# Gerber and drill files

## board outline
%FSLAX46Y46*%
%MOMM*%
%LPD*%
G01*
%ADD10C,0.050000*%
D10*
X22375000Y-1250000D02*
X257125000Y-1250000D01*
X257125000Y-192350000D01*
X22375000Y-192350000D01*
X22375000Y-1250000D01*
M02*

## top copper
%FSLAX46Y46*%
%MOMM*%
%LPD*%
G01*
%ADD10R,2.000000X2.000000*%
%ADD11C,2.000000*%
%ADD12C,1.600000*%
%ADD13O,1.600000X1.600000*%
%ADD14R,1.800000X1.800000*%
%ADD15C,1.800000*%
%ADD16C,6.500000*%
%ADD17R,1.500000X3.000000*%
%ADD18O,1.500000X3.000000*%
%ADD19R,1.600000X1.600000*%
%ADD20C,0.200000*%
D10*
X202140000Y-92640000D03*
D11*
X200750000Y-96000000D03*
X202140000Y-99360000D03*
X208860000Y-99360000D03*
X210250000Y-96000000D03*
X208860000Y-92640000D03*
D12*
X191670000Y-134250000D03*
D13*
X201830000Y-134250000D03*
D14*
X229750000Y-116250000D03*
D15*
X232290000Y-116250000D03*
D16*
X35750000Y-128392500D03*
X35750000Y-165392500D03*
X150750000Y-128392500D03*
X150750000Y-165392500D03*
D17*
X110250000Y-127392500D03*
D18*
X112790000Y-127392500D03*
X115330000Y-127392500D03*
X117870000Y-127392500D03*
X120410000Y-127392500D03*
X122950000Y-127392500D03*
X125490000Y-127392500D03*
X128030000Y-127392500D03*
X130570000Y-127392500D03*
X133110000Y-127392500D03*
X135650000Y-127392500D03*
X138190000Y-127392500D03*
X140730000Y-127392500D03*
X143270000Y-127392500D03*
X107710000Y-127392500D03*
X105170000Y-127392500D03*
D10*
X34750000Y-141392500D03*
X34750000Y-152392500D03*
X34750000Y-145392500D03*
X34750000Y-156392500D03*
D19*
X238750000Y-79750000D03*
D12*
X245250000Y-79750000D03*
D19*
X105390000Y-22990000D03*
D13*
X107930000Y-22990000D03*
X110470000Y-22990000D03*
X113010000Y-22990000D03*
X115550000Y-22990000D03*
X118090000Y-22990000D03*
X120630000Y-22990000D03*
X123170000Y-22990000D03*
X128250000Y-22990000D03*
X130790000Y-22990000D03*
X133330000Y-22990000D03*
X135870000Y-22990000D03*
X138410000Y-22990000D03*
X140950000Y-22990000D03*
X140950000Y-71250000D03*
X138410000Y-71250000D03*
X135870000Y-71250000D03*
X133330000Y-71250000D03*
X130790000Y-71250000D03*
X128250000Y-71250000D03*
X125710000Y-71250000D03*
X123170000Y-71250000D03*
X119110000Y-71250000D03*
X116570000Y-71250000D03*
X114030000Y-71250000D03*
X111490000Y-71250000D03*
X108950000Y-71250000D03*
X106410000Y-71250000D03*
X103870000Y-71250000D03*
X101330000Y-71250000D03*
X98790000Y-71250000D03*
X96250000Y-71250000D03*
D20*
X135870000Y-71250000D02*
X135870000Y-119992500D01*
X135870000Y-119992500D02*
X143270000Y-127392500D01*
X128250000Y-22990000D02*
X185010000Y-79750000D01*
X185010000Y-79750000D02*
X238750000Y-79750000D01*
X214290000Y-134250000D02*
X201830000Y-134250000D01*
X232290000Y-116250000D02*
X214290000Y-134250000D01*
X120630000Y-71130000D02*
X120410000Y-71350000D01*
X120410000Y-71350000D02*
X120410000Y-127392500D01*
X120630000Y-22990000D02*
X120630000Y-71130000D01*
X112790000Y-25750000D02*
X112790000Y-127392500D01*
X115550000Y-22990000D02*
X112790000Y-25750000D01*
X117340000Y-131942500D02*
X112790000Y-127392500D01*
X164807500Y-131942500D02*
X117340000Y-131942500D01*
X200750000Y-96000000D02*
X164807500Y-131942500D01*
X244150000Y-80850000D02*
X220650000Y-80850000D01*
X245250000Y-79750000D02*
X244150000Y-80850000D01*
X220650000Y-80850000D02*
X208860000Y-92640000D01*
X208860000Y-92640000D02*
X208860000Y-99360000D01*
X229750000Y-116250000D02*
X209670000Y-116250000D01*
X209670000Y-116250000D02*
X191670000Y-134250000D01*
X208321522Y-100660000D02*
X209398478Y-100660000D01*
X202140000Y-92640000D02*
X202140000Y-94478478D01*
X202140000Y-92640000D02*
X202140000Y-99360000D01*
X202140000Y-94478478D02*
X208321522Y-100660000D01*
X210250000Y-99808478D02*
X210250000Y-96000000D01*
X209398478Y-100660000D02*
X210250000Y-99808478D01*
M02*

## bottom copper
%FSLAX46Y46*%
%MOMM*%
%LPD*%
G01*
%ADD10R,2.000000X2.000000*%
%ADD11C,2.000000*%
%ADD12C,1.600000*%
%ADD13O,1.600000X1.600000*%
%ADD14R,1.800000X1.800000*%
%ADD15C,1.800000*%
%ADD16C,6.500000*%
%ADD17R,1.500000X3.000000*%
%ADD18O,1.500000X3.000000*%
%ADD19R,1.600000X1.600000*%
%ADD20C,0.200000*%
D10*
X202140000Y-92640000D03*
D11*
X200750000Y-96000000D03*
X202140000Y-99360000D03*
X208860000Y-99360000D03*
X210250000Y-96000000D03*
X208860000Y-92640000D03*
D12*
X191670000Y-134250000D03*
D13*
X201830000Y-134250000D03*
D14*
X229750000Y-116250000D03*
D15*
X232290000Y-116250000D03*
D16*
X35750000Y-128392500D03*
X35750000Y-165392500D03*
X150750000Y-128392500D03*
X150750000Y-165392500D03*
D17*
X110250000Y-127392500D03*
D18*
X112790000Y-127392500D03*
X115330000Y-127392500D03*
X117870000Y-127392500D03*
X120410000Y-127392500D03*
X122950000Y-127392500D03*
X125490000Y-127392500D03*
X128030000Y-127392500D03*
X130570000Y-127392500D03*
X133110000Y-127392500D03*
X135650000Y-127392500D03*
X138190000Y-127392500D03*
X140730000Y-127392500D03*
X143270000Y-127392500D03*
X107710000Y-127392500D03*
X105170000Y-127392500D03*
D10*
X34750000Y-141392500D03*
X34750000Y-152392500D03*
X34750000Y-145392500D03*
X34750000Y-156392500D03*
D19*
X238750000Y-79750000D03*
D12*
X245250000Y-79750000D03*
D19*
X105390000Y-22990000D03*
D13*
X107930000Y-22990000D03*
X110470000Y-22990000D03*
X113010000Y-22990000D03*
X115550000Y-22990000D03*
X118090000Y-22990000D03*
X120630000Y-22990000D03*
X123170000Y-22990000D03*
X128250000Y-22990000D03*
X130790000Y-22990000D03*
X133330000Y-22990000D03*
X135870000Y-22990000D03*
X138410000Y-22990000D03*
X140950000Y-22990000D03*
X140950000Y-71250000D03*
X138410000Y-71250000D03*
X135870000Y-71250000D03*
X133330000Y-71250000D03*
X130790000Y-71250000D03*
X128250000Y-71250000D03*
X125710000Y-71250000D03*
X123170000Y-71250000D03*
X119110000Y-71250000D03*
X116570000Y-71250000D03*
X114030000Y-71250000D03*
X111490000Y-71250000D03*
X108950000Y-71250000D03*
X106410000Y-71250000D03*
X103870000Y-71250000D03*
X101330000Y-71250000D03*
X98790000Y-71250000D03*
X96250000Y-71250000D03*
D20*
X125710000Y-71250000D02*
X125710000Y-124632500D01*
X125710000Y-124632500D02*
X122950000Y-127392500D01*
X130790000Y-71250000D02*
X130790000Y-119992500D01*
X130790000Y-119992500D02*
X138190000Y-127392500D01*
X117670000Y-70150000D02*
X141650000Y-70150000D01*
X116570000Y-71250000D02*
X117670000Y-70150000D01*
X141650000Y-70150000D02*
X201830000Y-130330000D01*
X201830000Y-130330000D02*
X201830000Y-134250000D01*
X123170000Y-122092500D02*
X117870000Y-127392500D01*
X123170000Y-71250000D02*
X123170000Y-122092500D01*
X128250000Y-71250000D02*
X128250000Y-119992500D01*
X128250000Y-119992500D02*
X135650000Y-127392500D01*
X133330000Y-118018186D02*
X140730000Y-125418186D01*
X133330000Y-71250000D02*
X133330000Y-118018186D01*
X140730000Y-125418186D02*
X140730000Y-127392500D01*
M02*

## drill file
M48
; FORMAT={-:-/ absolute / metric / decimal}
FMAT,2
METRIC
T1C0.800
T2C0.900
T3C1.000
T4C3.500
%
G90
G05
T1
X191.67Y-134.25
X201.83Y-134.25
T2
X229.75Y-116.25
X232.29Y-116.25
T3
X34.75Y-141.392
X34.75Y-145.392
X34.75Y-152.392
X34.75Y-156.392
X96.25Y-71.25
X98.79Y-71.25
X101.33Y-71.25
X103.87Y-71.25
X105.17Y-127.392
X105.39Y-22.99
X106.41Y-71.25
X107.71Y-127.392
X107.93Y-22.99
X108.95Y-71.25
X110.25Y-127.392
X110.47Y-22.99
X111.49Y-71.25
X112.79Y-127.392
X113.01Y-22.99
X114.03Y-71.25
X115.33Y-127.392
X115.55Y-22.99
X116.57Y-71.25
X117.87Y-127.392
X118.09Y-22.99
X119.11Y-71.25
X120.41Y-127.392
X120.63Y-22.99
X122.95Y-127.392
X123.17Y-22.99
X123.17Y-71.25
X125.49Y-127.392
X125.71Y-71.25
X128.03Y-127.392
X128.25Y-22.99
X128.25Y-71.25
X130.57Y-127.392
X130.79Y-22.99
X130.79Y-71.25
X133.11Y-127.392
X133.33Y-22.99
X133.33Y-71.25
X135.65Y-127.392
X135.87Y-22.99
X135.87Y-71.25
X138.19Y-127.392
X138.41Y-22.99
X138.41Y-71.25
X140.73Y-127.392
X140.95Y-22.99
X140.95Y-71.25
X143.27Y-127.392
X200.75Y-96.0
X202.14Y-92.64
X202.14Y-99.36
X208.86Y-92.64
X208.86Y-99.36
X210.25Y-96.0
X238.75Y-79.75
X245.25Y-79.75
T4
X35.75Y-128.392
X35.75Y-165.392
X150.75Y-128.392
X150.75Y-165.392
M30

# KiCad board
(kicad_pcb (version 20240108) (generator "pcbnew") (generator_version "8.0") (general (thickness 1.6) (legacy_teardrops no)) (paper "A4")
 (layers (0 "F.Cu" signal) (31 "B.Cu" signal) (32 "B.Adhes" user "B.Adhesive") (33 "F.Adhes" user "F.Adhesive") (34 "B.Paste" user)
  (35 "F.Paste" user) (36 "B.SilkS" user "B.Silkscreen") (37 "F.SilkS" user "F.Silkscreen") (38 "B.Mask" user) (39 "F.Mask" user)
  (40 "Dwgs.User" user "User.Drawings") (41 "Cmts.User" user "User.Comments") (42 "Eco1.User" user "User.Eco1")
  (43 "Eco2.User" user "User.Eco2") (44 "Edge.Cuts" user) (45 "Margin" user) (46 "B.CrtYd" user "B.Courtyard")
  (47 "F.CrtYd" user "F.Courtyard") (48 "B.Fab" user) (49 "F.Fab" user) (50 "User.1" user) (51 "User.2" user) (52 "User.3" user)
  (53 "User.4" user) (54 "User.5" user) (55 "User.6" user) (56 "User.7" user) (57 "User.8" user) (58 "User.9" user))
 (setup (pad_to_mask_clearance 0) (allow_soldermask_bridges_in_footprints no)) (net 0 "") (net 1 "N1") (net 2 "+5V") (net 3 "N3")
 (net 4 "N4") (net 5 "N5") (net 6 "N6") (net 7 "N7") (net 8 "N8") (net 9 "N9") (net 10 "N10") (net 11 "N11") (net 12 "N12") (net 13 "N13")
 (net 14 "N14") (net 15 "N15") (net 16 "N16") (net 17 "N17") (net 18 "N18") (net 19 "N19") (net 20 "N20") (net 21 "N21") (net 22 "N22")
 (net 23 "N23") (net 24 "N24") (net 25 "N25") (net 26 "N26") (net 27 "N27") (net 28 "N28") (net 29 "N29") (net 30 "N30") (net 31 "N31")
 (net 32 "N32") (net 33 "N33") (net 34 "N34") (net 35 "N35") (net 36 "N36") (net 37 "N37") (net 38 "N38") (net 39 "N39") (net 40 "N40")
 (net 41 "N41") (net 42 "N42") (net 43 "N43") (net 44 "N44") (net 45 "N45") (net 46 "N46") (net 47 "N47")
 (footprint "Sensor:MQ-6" (layer "F.Cu") (at 202.14 92.64)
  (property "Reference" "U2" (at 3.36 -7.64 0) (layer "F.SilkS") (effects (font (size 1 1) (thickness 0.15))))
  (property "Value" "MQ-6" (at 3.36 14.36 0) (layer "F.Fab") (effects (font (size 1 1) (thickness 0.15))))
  (pad "1" thru_hole rect (at 0 0) (size 2 2) (drill 1) (layers "*.Cu" "*.Mask") (remove_unused_layers no) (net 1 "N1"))
  (pad "2" thru_hole circle (at -1.39 3.36) (size 2 2) (drill 1) (layers "*.Cu" "*.Mask") (remove_unused_layers no) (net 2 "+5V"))
  (pad "3" thru_hole circle (at 0 6.72 90) (size 2 2) (drill 1) (layers "*.Cu" "*.Mask") (remove_unused_layers no) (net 1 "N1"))
  (pad "4" thru_hole circle (at 6.72 6.72 180) (size 2 2) (drill 1) (layers "*.Cu" "*.Mask") (remove_unused_layers no) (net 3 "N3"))
  (pad "5" thru_hole circle (at 8.11 3.36) (size 2 2) (drill 1) (layers "*.Cu" "*.Mask") (remove_unused_layers no) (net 1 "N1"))
  (pad "6" thru_hole circle (at 6.72 0 270) (size 2 2) (drill 1) (layers "*.Cu" "*.Mask") (remove_unused_layers no) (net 3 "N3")))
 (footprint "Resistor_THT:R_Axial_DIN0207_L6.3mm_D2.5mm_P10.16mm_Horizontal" (layer "F.Cu") (at 191.67 134.25)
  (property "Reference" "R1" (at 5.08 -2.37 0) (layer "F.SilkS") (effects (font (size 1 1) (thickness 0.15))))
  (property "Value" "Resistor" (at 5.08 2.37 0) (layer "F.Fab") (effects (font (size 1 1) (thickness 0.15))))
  (pad "1" thru_hole circle (at 0 0) (size 1.6 1.6) (drill 0.8) (layers "*.Cu" "*.Mask") (remove_unused_layers no) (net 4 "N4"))
  (pad "2" thru_hole oval (at 10.16 0) (size 1.6 1.6) (drill 0.8) (layers "*.Cu" "*.Mask") (remove_unused_layers no) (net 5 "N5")))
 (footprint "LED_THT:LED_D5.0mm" (layer "F.Cu") (at 229.75 116.25)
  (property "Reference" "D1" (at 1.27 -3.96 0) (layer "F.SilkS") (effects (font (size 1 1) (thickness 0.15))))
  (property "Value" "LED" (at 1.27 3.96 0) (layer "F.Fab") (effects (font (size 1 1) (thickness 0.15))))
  (pad "1" thru_hole rect (at 0 0) (size 1.8 1.8) (drill 0.9) (layers "*.Cu" "*.Mask") (remove_unused_layers no) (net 4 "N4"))
  (pad "2" thru_hole circle (at 2.54 0) (size 1.8 1.8) (drill 0.9) (layers "*.Cu" "*.Mask") (remove_unused_layers no) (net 5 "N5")))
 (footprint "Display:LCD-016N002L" (layer "F.Cu") (at 110.25 127.3925)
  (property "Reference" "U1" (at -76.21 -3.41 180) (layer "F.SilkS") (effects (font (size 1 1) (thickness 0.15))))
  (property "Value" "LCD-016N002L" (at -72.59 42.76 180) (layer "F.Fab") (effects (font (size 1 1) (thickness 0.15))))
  (pad "" thru_hole circle (at -74.5 1 180) (size 6.5 6.5) (drill 3.5) (layers "*.Cu" "*.Mask") (remove_unused_layers no))
  (pad "" thru_hole circle (at -74.5 38 180) (size 6.5 6.5) (drill 3.5) (layers "*.Cu" "*.Mask") (remove_unused_layers no))
  (pad "" thru_hole circle (at 40.5 1 180) (size 6.5 6.5) (drill 3.5) (layers "*.Cu" "*.Mask") (remove_unused_layers no))
  (pad "" thru_hole circle (at 40.5 38 180) (size 6.5 6.5) (drill 3.5) (layers "*.Cu" "*.Mask") (remove_unused_layers no))
  (pad "1" thru_hole rect (at 0 0 180) (size 1.5 3) (drill 1) (layers "*.Cu" "*.Mask") (remove_unused_layers no) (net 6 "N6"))
  (pad "2" thru_hole oval (at 2.54 0 180) (size 1.5 3) (drill 1) (layers "*.Cu" "*.Mask") (remove_unused_layers no) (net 2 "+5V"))
  (pad "3" thru_hole oval (at 5.08 0 180) (size 1.5 3) (drill 1) (layers "*.Cu" "*.Mask") (remove_unused_layers no) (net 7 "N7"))
  (pad "4" thru_hole oval (at 7.62 0 180) (size 1.5 3) (drill 1) (layers "*.Cu" "*.Mask") (remove_unused_layers no) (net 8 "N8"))
  (pad "5" thru_hole oval (at 10.16 0 180) (size 1.5 3) (drill 1) (layers "*.Cu" "*.Mask") (remove_unused_layers no) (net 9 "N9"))
  (pad "6" thru_hole oval (at 12.7 0 180) (size 1.5 3) (drill 1) (layers "*.Cu" "*.Mask") (remove_unused_layers no) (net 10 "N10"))
  (pad "7" thru_hole oval (at 15.24 0 180) (size 1.5 3) (drill 1) (layers "*.Cu" "*.Mask") (remove_unused_layers no) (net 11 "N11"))
  (pad "8" thru_hole oval (at 17.78 0 180) (size 1.5 3) (drill 1) (layers "*.Cu" "*.Mask") (remove_unused_layers no) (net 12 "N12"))
  (pad "9" thru_hole oval (at 20.32 0 180) (size 1.5 3) (drill 1) (layers "*.Cu" "*.Mask") (remove_unused_layers no) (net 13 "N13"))
  (pad "10" thru_hole oval (at 22.86 0 180) (size 1.5 3) (drill 1) (layers "*.Cu" "*.Mask") (remove_unused_layers no) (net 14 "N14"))
  (pad "11" thru_hole oval (at 25.4 0 180) (size 1.5 3) (drill 1) (layers "*.Cu" "*.Mask") (remove_unused_layers no) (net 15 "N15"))
  (pad "12" thru_hole oval (at 27.94 0 180) (size 1.5 3) (drill 1) (layers "*.Cu" "*.Mask") (remove_unused_layers no) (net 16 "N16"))
  (pad "13" thru_hole oval (at 30.48 0 180) (size 1.5 3) (drill 1) (layers "*.Cu" "*.Mask") (remove_unused_layers no) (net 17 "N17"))
  (pad "14" thru_hole oval (at 33.02 0 180) (size 1.5 3) (drill 1) (layers "*.Cu" "*.Mask") (remove_unused_layers no) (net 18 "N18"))
  (pad "15" thru_hole oval (at -2.54 0 180) (size 1.5 3) (drill 1) (layers "*.Cu" "*.Mask") (remove_unused_layers no) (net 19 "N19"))
  (pad "16" thru_hole oval (at -5.08 0 180) (size 1.5 3) (drill 1) (layers "*.Cu" "*.Mask") (remove_unused_layers no) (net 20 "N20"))
  (pad "A1" thru_hole rect (at -75.5 14 180) (size 2 2) (drill 1) (layers "*.Cu" "*.Mask") (remove_unused_layers no) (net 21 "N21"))
  (pad "A2" thru_hole rect (at -75.5 25 180) (size 2 2) (drill 1) (layers "*.Cu" "*.Mask") (remove_unused_layers no) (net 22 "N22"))
  (pad "K1" thru_hole rect (at -75.5 18 180) (size 2 2) (drill 1) (layers "*.Cu" "*.Mask") (remove_unused_layers no) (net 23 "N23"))
  (pad "K2" thru_hole rect (at -75.5 29 180) (size 2 2) (drill 1) (layers "*.Cu" "*.Mask") (remove_unused_layers no) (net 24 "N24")))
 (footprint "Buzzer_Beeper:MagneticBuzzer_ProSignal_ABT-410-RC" (layer "F.Cu") (at 238.75 79.75)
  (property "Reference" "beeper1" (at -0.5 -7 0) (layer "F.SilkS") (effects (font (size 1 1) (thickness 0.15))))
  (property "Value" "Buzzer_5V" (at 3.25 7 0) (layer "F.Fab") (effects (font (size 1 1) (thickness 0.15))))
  (pad "1" thru_hole rect (at 0 0) (size 1.6 1.6) (drill 1) (layers "*.Cu" "*.Mask") (remove_unused_layers no) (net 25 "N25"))
  (pad "2" thru_hole circle (at 6.5 0) (size 1.6 1.6) (drill 1) (layers "*.Cu" "*.Mask") (remove_unused_layers no) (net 3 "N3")))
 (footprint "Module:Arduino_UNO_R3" (layer "F.Cu") (at 105.39 22.99)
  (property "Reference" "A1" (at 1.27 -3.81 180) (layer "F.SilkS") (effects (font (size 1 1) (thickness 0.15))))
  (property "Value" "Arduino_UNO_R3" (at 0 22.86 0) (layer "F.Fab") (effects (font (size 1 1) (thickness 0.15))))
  (pad "1" thru_hole rect (at 0 0 90) (size 1.6 1.6) (drill 1) (layers "*.Cu" "*.Mask") (remove_unused_layers no) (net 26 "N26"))
  (pad "2" thru_hole oval (at 2.54 0 90) (size 1.6 1.6) (drill 1) (layers "*.Cu" "*.Mask") (remove_unused_layers no) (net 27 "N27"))
  (pad "3" thru_hole oval (at 5.08 0 90) (size 1.6 1.6) (drill 1) (layers "*.Cu" "*.Mask") (remove_unused_layers no) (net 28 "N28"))
  (pad "4" thru_hole oval (at 7.62 0 90) (size 1.6 1.6) (drill 1) (layers "*.Cu" "*.Mask") (remove_unused_layers no) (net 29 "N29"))
  (pad "5" thru_hole oval (at 10.16 0 90) (size 1.6 1.6) (drill 1) (layers "*.Cu" "*.Mask") (remove_unused_layers no) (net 2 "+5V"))
  (pad "6" thru_hole oval (at 12.7 0 90) (size 1.6 1.6) (drill 1) (layers "*.Cu" "*.Mask") (remove_unused_layers no) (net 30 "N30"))
  (pad "7" thru_hole oval (at 15.24 0 90) (size 1.6 1.6) (drill 1) (layers "*.Cu" "*.Mask") (remove_unused_layers no) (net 9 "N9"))
  (pad "8" thru_hole oval (at 17.78 0 90) (size 1.6 1.6) (drill 1) (layers "*.Cu" "*.Mask") (remove_unused_layers no) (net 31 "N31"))
  (pad "9" thru_hole oval (at 22.86 0 90) (size 1.6 1.6) (drill 1) (layers "*.Cu" "*.Mask") (remove_unused_layers no) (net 25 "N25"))
  (pad "10" thru_hole oval (at 25.4 0 90) (size 1.6 1.6) (drill 1) (layers "*.Cu" "*.Mask") (remove_unused_layers no) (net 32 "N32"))
  (pad "11" thru_hole oval (at 27.94 0 90) (size 1.6 1.6) (drill 1) (layers "*.Cu" "*.Mask") (remove_unused_layers no) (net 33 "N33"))
  (pad "12" thru_hole oval (at 30.48 0 90) (size 1.6 1.6) (drill 1) (layers "*.Cu" "*.Mask") (remove_unused_layers no) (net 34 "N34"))
  (pad "13" thru_hole oval (at 33.02 0 90) (size 1.6 1.6) (drill 1) (layers "*.Cu" "*.Mask") (remove_unused_layers no) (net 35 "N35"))
  (pad "14" thru_hole oval (at 35.56 0 90) (size 1.6 1.6) (drill 1) (layers "*.Cu" "*.Mask") (remove_unused_layers no) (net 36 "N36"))
  (pad "15" thru_hole oval (at 35.56 48.26 90) (size 1.6 1.6) (drill 1) (layers "*.Cu" "*.Mask") (remove_unused_layers no) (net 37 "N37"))
  (pad "16" thru_hole oval (at 33.02 48.26 90) (size 1.6 1.6) (drill 1) (layers "*.Cu" "*.Mask") (remove_unused_layers no) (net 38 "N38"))
  (pad "17" thru_hole oval (at 30.48 48.26 90) (size 1.6 1.6) (drill 1) (layers "*.Cu" "*.Mask") (remove_unused_layers no) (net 18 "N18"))
  (pad "18" thru_hole oval (at 27.94 48.26 90) (size 1.6 1.6) (drill 1) (layers "*.Cu" "*.Mask") (remove_unused_layers no) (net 17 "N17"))
  (pad "19" thru_hole oval (at 25.4 48.26 90) (size 1.6 1.6) (drill 1) (layers "*.Cu" "*.Mask") (remove_unused_layers no) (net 16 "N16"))
  (pad "20" thru_hole oval (at 22.86 48.26 90) (size 1.6 1.6) (drill 1) (layers "*.Cu" "*.Mask") (remove_unused_layers no) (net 15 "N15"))
  (pad "21" thru_hole oval (at 20.32 48.26 90) (size 1.6 1.6) (drill 1) (layers "*.Cu" "*.Mask") (remove_unused_layers no) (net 10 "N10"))
  (pad "22" thru_hole oval (at 17.78 48.26 90) (size 1.6 1.6) (drill 1) (layers "*.Cu" "*.Mask") (remove_unused_layers no) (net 8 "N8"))
  (pad "23" thru_hole oval (at 13.72 48.26 90) (size 1.6 1.6) (drill 1) (layers "*.Cu" "*.Mask") (remove_unused_layers no) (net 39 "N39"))
  (pad "24" thru_hole oval (at 11.18 48.26 90) (size 1.6 1.6) (drill 1) (layers "*.Cu" "*.Mask") (remove_unused_layers no) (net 5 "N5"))
  (pad "25" thru_hole oval (at 8.64 48.26 90) (size 1.6 1.6) (drill 1) (layers "*.Cu" "*.Mask") (remove_unused_layers no) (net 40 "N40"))
  (pad "26" thru_hole oval (at 6.1 48.26 90) (size 1.6 1.6) (drill 1) (layers "*.Cu" "*.Mask") (remove_unused_layers no) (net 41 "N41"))
  (pad "27" thru_hole oval (at 3.56 48.26 90) (size 1.6 1.6) (drill 1) (layers "*.Cu" "*.Mask") (remove_unused_layers no) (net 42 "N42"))
  (pad "28" thru_hole oval (at 1.02 48.26 90) (size 1.6 1.6) (drill 1) (layers "*.Cu" "*.Mask") (remove_unused_layers no) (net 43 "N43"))
  (pad "29" thru_hole oval (at -1.52 48.26 90) (size 1.6 1.6) (drill 1) (layers "*.Cu" "*.Mask") (remove_unused_layers no) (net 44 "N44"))
  (pad "30" thru_hole oval (at -4.06 48.26 90) (size 1.6 1.6) (drill 1) (layers "*.Cu" "*.Mask") (remove_unused_layers no) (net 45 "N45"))
  (pad "31" thru_hole oval (at -6.6 48.26 90) (size 1.6 1.6) (drill 1) (layers "*.Cu" "*.Mask") (remove_unused_layers no) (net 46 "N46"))
  (pad "32" thru_hole oval (at -9.14 48.26 90) (size 1.6 1.6) (drill 1) (layers "*.Cu" "*.Mask") (remove_unused_layers no) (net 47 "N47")))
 (gr_rect (start 22.375 1.25) (end 257.125 192.35) (stroke (width 0.05) (type default)) (fill none) (layer "Edge.Cuts"))
 (segment (start 125.71 71.25) (end 125.71 124.6325) (width 0.2) (layer "B.Cu") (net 10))
 (segment (start 125.71 124.6325) (end 122.95 127.3925) (width 0.2) (layer "B.Cu") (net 10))
 (segment (start 135.87 71.25) (end 135.87 119.9925) (width 0.2) (layer "F.Cu") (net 18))
 (segment (start 135.87 119.9925) (end 143.27 127.3925) (width 0.2) (layer "F.Cu") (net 18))
 (segment (start 130.79 71.25) (end 130.79 119.9925) (width 0.2) (layer "B.Cu") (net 16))
 (segment (start 130.79 119.9925) (end 138.19 127.3925) (width 0.2) (layer "B.Cu") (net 16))
 (segment (start 128.25 22.99) (end 185.01 79.75) (width 0.2) (layer "F.Cu") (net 25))
 (segment (start 185.01 79.75) (end 238.75 79.75) (width 0.2) (layer "F.Cu") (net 25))
 (segment (start 214.29 134.25) (end 201.83 134.25) (width 0.2) (layer "F.Cu") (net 5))
 (segment (start 232.29 116.25) (end 214.29 134.25) (width 0.2) (layer "F.Cu") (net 5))
 (segment (start 117.67 70.15) (end 141.65 70.15) (width 0.2) (layer "B.Cu") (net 5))
 (segment (start 116.57 71.25) (end 117.67 70.15) (width 0.2) (layer "B.Cu") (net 5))
 (segment (start 141.65 70.15) (end 201.83 130.33) (width 0.2) (layer "B.Cu") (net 5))
 (segment (start 201.83 130.33) (end 201.83 134.25) (width 0.2) (layer "B.Cu") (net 5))
 (segment (start 123.17 122.0925) (end 117.87 127.3925) (width 0.2) (layer "B.Cu") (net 8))
 (segment (start 123.17 71.25) (end 123.17 122.0925) (width 0.2) (layer "B.Cu") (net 8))
 (segment (start 128.25 71.25) (end 128.25 119.9925) (width 0.2) (layer "B.Cu") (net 15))
 (segment (start 128.25 119.9925) (end 135.65 127.3925) (width 0.2) (layer "B.Cu") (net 15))
 (segment (start 120.63 71.13) (end 120.41 71.35) (width 0.2) (layer "F.Cu") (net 9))
 (segment (start 120.41 71.35) (end 120.41 127.3925) (width 0.2) (layer "F.Cu") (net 9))
 (segment (start 120.63 22.99) (end 120.63 71.13) (width 0.2) (layer "F.Cu") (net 9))
 (segment (start 133.33 118.018186) (end 140.73 125.418186) (width 0.2) (layer "B.Cu") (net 17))
 (segment (start 133.33 71.25) (end 133.33 118.018186) (width 0.2) (layer "B.Cu") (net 17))
 (segment (start 140.73 125.418186) (end 140.73 127.3925) (width 0.2) (layer "B.Cu") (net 17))
 (segment (start 112.79 25.75) (end 112.79 127.3925) (width 0.2) (layer "F.Cu") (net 2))
 (segment (start 115.55 22.99) (end 112.79 25.75) (width 0.2) (layer "F.Cu") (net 2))
 (segment (start 117.34 131.9425) (end 112.79 127.3925) (width 0.2) (layer "F.Cu") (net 2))
 (segment (start 164.8075 131.9425) (end 117.34 131.9425) (width 0.2) (layer "F.Cu") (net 2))
 (segment (start 200.75 96) (end 164.8075 131.9425) (width 0.2) (layer "F.Cu") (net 2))
 (segment (start 244.15 80.85) (end 220.65 80.85) (width 0.2) (layer "F.Cu") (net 3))
 (segment (start 245.25 79.75) (end 244.15 80.85) (width 0.2) (layer "F.Cu") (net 3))
 (segment (start 220.65 80.85) (end 208.86 92.64) (width 0.2) (layer "F.Cu") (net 3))
 (segment (start 208.86 92.64) (end 208.86 99.36) (width 0.2) (layer "F.Cu") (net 3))
 (segment (start 229.75 116.25) (end 209.67 116.25) (width 0.2) (layer "F.Cu") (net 4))
 (segment (start 209.67 116.25) (end 191.67 134.25) (width 0.2) (layer "F.Cu") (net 4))
 (segment (start 208.321522 100.66) (end 209.398478 100.66) (width 0.2) (layer "F.Cu") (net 1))
 (segment (start 202.14 92.64) (end 202.14 94.478478) (width 0.2) (layer "F.Cu") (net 1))
 (segment (start 202.14 92.64) (end 202.14 99.36) (width 0.2) (layer "F.Cu") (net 1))
 (segment (start 202.14 94.478478) (end 208.321522 100.66) (width 0.2) (layer "F.Cu") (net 1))
 (segment (start 210.25 99.808478) (end 210.25 96) (width 0.2) (layer "F.Cu") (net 1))
 (segment (start 209.398478 100.66) (end 210.25 99.808478) (width 0.2) (layer "F.Cu") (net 1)))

